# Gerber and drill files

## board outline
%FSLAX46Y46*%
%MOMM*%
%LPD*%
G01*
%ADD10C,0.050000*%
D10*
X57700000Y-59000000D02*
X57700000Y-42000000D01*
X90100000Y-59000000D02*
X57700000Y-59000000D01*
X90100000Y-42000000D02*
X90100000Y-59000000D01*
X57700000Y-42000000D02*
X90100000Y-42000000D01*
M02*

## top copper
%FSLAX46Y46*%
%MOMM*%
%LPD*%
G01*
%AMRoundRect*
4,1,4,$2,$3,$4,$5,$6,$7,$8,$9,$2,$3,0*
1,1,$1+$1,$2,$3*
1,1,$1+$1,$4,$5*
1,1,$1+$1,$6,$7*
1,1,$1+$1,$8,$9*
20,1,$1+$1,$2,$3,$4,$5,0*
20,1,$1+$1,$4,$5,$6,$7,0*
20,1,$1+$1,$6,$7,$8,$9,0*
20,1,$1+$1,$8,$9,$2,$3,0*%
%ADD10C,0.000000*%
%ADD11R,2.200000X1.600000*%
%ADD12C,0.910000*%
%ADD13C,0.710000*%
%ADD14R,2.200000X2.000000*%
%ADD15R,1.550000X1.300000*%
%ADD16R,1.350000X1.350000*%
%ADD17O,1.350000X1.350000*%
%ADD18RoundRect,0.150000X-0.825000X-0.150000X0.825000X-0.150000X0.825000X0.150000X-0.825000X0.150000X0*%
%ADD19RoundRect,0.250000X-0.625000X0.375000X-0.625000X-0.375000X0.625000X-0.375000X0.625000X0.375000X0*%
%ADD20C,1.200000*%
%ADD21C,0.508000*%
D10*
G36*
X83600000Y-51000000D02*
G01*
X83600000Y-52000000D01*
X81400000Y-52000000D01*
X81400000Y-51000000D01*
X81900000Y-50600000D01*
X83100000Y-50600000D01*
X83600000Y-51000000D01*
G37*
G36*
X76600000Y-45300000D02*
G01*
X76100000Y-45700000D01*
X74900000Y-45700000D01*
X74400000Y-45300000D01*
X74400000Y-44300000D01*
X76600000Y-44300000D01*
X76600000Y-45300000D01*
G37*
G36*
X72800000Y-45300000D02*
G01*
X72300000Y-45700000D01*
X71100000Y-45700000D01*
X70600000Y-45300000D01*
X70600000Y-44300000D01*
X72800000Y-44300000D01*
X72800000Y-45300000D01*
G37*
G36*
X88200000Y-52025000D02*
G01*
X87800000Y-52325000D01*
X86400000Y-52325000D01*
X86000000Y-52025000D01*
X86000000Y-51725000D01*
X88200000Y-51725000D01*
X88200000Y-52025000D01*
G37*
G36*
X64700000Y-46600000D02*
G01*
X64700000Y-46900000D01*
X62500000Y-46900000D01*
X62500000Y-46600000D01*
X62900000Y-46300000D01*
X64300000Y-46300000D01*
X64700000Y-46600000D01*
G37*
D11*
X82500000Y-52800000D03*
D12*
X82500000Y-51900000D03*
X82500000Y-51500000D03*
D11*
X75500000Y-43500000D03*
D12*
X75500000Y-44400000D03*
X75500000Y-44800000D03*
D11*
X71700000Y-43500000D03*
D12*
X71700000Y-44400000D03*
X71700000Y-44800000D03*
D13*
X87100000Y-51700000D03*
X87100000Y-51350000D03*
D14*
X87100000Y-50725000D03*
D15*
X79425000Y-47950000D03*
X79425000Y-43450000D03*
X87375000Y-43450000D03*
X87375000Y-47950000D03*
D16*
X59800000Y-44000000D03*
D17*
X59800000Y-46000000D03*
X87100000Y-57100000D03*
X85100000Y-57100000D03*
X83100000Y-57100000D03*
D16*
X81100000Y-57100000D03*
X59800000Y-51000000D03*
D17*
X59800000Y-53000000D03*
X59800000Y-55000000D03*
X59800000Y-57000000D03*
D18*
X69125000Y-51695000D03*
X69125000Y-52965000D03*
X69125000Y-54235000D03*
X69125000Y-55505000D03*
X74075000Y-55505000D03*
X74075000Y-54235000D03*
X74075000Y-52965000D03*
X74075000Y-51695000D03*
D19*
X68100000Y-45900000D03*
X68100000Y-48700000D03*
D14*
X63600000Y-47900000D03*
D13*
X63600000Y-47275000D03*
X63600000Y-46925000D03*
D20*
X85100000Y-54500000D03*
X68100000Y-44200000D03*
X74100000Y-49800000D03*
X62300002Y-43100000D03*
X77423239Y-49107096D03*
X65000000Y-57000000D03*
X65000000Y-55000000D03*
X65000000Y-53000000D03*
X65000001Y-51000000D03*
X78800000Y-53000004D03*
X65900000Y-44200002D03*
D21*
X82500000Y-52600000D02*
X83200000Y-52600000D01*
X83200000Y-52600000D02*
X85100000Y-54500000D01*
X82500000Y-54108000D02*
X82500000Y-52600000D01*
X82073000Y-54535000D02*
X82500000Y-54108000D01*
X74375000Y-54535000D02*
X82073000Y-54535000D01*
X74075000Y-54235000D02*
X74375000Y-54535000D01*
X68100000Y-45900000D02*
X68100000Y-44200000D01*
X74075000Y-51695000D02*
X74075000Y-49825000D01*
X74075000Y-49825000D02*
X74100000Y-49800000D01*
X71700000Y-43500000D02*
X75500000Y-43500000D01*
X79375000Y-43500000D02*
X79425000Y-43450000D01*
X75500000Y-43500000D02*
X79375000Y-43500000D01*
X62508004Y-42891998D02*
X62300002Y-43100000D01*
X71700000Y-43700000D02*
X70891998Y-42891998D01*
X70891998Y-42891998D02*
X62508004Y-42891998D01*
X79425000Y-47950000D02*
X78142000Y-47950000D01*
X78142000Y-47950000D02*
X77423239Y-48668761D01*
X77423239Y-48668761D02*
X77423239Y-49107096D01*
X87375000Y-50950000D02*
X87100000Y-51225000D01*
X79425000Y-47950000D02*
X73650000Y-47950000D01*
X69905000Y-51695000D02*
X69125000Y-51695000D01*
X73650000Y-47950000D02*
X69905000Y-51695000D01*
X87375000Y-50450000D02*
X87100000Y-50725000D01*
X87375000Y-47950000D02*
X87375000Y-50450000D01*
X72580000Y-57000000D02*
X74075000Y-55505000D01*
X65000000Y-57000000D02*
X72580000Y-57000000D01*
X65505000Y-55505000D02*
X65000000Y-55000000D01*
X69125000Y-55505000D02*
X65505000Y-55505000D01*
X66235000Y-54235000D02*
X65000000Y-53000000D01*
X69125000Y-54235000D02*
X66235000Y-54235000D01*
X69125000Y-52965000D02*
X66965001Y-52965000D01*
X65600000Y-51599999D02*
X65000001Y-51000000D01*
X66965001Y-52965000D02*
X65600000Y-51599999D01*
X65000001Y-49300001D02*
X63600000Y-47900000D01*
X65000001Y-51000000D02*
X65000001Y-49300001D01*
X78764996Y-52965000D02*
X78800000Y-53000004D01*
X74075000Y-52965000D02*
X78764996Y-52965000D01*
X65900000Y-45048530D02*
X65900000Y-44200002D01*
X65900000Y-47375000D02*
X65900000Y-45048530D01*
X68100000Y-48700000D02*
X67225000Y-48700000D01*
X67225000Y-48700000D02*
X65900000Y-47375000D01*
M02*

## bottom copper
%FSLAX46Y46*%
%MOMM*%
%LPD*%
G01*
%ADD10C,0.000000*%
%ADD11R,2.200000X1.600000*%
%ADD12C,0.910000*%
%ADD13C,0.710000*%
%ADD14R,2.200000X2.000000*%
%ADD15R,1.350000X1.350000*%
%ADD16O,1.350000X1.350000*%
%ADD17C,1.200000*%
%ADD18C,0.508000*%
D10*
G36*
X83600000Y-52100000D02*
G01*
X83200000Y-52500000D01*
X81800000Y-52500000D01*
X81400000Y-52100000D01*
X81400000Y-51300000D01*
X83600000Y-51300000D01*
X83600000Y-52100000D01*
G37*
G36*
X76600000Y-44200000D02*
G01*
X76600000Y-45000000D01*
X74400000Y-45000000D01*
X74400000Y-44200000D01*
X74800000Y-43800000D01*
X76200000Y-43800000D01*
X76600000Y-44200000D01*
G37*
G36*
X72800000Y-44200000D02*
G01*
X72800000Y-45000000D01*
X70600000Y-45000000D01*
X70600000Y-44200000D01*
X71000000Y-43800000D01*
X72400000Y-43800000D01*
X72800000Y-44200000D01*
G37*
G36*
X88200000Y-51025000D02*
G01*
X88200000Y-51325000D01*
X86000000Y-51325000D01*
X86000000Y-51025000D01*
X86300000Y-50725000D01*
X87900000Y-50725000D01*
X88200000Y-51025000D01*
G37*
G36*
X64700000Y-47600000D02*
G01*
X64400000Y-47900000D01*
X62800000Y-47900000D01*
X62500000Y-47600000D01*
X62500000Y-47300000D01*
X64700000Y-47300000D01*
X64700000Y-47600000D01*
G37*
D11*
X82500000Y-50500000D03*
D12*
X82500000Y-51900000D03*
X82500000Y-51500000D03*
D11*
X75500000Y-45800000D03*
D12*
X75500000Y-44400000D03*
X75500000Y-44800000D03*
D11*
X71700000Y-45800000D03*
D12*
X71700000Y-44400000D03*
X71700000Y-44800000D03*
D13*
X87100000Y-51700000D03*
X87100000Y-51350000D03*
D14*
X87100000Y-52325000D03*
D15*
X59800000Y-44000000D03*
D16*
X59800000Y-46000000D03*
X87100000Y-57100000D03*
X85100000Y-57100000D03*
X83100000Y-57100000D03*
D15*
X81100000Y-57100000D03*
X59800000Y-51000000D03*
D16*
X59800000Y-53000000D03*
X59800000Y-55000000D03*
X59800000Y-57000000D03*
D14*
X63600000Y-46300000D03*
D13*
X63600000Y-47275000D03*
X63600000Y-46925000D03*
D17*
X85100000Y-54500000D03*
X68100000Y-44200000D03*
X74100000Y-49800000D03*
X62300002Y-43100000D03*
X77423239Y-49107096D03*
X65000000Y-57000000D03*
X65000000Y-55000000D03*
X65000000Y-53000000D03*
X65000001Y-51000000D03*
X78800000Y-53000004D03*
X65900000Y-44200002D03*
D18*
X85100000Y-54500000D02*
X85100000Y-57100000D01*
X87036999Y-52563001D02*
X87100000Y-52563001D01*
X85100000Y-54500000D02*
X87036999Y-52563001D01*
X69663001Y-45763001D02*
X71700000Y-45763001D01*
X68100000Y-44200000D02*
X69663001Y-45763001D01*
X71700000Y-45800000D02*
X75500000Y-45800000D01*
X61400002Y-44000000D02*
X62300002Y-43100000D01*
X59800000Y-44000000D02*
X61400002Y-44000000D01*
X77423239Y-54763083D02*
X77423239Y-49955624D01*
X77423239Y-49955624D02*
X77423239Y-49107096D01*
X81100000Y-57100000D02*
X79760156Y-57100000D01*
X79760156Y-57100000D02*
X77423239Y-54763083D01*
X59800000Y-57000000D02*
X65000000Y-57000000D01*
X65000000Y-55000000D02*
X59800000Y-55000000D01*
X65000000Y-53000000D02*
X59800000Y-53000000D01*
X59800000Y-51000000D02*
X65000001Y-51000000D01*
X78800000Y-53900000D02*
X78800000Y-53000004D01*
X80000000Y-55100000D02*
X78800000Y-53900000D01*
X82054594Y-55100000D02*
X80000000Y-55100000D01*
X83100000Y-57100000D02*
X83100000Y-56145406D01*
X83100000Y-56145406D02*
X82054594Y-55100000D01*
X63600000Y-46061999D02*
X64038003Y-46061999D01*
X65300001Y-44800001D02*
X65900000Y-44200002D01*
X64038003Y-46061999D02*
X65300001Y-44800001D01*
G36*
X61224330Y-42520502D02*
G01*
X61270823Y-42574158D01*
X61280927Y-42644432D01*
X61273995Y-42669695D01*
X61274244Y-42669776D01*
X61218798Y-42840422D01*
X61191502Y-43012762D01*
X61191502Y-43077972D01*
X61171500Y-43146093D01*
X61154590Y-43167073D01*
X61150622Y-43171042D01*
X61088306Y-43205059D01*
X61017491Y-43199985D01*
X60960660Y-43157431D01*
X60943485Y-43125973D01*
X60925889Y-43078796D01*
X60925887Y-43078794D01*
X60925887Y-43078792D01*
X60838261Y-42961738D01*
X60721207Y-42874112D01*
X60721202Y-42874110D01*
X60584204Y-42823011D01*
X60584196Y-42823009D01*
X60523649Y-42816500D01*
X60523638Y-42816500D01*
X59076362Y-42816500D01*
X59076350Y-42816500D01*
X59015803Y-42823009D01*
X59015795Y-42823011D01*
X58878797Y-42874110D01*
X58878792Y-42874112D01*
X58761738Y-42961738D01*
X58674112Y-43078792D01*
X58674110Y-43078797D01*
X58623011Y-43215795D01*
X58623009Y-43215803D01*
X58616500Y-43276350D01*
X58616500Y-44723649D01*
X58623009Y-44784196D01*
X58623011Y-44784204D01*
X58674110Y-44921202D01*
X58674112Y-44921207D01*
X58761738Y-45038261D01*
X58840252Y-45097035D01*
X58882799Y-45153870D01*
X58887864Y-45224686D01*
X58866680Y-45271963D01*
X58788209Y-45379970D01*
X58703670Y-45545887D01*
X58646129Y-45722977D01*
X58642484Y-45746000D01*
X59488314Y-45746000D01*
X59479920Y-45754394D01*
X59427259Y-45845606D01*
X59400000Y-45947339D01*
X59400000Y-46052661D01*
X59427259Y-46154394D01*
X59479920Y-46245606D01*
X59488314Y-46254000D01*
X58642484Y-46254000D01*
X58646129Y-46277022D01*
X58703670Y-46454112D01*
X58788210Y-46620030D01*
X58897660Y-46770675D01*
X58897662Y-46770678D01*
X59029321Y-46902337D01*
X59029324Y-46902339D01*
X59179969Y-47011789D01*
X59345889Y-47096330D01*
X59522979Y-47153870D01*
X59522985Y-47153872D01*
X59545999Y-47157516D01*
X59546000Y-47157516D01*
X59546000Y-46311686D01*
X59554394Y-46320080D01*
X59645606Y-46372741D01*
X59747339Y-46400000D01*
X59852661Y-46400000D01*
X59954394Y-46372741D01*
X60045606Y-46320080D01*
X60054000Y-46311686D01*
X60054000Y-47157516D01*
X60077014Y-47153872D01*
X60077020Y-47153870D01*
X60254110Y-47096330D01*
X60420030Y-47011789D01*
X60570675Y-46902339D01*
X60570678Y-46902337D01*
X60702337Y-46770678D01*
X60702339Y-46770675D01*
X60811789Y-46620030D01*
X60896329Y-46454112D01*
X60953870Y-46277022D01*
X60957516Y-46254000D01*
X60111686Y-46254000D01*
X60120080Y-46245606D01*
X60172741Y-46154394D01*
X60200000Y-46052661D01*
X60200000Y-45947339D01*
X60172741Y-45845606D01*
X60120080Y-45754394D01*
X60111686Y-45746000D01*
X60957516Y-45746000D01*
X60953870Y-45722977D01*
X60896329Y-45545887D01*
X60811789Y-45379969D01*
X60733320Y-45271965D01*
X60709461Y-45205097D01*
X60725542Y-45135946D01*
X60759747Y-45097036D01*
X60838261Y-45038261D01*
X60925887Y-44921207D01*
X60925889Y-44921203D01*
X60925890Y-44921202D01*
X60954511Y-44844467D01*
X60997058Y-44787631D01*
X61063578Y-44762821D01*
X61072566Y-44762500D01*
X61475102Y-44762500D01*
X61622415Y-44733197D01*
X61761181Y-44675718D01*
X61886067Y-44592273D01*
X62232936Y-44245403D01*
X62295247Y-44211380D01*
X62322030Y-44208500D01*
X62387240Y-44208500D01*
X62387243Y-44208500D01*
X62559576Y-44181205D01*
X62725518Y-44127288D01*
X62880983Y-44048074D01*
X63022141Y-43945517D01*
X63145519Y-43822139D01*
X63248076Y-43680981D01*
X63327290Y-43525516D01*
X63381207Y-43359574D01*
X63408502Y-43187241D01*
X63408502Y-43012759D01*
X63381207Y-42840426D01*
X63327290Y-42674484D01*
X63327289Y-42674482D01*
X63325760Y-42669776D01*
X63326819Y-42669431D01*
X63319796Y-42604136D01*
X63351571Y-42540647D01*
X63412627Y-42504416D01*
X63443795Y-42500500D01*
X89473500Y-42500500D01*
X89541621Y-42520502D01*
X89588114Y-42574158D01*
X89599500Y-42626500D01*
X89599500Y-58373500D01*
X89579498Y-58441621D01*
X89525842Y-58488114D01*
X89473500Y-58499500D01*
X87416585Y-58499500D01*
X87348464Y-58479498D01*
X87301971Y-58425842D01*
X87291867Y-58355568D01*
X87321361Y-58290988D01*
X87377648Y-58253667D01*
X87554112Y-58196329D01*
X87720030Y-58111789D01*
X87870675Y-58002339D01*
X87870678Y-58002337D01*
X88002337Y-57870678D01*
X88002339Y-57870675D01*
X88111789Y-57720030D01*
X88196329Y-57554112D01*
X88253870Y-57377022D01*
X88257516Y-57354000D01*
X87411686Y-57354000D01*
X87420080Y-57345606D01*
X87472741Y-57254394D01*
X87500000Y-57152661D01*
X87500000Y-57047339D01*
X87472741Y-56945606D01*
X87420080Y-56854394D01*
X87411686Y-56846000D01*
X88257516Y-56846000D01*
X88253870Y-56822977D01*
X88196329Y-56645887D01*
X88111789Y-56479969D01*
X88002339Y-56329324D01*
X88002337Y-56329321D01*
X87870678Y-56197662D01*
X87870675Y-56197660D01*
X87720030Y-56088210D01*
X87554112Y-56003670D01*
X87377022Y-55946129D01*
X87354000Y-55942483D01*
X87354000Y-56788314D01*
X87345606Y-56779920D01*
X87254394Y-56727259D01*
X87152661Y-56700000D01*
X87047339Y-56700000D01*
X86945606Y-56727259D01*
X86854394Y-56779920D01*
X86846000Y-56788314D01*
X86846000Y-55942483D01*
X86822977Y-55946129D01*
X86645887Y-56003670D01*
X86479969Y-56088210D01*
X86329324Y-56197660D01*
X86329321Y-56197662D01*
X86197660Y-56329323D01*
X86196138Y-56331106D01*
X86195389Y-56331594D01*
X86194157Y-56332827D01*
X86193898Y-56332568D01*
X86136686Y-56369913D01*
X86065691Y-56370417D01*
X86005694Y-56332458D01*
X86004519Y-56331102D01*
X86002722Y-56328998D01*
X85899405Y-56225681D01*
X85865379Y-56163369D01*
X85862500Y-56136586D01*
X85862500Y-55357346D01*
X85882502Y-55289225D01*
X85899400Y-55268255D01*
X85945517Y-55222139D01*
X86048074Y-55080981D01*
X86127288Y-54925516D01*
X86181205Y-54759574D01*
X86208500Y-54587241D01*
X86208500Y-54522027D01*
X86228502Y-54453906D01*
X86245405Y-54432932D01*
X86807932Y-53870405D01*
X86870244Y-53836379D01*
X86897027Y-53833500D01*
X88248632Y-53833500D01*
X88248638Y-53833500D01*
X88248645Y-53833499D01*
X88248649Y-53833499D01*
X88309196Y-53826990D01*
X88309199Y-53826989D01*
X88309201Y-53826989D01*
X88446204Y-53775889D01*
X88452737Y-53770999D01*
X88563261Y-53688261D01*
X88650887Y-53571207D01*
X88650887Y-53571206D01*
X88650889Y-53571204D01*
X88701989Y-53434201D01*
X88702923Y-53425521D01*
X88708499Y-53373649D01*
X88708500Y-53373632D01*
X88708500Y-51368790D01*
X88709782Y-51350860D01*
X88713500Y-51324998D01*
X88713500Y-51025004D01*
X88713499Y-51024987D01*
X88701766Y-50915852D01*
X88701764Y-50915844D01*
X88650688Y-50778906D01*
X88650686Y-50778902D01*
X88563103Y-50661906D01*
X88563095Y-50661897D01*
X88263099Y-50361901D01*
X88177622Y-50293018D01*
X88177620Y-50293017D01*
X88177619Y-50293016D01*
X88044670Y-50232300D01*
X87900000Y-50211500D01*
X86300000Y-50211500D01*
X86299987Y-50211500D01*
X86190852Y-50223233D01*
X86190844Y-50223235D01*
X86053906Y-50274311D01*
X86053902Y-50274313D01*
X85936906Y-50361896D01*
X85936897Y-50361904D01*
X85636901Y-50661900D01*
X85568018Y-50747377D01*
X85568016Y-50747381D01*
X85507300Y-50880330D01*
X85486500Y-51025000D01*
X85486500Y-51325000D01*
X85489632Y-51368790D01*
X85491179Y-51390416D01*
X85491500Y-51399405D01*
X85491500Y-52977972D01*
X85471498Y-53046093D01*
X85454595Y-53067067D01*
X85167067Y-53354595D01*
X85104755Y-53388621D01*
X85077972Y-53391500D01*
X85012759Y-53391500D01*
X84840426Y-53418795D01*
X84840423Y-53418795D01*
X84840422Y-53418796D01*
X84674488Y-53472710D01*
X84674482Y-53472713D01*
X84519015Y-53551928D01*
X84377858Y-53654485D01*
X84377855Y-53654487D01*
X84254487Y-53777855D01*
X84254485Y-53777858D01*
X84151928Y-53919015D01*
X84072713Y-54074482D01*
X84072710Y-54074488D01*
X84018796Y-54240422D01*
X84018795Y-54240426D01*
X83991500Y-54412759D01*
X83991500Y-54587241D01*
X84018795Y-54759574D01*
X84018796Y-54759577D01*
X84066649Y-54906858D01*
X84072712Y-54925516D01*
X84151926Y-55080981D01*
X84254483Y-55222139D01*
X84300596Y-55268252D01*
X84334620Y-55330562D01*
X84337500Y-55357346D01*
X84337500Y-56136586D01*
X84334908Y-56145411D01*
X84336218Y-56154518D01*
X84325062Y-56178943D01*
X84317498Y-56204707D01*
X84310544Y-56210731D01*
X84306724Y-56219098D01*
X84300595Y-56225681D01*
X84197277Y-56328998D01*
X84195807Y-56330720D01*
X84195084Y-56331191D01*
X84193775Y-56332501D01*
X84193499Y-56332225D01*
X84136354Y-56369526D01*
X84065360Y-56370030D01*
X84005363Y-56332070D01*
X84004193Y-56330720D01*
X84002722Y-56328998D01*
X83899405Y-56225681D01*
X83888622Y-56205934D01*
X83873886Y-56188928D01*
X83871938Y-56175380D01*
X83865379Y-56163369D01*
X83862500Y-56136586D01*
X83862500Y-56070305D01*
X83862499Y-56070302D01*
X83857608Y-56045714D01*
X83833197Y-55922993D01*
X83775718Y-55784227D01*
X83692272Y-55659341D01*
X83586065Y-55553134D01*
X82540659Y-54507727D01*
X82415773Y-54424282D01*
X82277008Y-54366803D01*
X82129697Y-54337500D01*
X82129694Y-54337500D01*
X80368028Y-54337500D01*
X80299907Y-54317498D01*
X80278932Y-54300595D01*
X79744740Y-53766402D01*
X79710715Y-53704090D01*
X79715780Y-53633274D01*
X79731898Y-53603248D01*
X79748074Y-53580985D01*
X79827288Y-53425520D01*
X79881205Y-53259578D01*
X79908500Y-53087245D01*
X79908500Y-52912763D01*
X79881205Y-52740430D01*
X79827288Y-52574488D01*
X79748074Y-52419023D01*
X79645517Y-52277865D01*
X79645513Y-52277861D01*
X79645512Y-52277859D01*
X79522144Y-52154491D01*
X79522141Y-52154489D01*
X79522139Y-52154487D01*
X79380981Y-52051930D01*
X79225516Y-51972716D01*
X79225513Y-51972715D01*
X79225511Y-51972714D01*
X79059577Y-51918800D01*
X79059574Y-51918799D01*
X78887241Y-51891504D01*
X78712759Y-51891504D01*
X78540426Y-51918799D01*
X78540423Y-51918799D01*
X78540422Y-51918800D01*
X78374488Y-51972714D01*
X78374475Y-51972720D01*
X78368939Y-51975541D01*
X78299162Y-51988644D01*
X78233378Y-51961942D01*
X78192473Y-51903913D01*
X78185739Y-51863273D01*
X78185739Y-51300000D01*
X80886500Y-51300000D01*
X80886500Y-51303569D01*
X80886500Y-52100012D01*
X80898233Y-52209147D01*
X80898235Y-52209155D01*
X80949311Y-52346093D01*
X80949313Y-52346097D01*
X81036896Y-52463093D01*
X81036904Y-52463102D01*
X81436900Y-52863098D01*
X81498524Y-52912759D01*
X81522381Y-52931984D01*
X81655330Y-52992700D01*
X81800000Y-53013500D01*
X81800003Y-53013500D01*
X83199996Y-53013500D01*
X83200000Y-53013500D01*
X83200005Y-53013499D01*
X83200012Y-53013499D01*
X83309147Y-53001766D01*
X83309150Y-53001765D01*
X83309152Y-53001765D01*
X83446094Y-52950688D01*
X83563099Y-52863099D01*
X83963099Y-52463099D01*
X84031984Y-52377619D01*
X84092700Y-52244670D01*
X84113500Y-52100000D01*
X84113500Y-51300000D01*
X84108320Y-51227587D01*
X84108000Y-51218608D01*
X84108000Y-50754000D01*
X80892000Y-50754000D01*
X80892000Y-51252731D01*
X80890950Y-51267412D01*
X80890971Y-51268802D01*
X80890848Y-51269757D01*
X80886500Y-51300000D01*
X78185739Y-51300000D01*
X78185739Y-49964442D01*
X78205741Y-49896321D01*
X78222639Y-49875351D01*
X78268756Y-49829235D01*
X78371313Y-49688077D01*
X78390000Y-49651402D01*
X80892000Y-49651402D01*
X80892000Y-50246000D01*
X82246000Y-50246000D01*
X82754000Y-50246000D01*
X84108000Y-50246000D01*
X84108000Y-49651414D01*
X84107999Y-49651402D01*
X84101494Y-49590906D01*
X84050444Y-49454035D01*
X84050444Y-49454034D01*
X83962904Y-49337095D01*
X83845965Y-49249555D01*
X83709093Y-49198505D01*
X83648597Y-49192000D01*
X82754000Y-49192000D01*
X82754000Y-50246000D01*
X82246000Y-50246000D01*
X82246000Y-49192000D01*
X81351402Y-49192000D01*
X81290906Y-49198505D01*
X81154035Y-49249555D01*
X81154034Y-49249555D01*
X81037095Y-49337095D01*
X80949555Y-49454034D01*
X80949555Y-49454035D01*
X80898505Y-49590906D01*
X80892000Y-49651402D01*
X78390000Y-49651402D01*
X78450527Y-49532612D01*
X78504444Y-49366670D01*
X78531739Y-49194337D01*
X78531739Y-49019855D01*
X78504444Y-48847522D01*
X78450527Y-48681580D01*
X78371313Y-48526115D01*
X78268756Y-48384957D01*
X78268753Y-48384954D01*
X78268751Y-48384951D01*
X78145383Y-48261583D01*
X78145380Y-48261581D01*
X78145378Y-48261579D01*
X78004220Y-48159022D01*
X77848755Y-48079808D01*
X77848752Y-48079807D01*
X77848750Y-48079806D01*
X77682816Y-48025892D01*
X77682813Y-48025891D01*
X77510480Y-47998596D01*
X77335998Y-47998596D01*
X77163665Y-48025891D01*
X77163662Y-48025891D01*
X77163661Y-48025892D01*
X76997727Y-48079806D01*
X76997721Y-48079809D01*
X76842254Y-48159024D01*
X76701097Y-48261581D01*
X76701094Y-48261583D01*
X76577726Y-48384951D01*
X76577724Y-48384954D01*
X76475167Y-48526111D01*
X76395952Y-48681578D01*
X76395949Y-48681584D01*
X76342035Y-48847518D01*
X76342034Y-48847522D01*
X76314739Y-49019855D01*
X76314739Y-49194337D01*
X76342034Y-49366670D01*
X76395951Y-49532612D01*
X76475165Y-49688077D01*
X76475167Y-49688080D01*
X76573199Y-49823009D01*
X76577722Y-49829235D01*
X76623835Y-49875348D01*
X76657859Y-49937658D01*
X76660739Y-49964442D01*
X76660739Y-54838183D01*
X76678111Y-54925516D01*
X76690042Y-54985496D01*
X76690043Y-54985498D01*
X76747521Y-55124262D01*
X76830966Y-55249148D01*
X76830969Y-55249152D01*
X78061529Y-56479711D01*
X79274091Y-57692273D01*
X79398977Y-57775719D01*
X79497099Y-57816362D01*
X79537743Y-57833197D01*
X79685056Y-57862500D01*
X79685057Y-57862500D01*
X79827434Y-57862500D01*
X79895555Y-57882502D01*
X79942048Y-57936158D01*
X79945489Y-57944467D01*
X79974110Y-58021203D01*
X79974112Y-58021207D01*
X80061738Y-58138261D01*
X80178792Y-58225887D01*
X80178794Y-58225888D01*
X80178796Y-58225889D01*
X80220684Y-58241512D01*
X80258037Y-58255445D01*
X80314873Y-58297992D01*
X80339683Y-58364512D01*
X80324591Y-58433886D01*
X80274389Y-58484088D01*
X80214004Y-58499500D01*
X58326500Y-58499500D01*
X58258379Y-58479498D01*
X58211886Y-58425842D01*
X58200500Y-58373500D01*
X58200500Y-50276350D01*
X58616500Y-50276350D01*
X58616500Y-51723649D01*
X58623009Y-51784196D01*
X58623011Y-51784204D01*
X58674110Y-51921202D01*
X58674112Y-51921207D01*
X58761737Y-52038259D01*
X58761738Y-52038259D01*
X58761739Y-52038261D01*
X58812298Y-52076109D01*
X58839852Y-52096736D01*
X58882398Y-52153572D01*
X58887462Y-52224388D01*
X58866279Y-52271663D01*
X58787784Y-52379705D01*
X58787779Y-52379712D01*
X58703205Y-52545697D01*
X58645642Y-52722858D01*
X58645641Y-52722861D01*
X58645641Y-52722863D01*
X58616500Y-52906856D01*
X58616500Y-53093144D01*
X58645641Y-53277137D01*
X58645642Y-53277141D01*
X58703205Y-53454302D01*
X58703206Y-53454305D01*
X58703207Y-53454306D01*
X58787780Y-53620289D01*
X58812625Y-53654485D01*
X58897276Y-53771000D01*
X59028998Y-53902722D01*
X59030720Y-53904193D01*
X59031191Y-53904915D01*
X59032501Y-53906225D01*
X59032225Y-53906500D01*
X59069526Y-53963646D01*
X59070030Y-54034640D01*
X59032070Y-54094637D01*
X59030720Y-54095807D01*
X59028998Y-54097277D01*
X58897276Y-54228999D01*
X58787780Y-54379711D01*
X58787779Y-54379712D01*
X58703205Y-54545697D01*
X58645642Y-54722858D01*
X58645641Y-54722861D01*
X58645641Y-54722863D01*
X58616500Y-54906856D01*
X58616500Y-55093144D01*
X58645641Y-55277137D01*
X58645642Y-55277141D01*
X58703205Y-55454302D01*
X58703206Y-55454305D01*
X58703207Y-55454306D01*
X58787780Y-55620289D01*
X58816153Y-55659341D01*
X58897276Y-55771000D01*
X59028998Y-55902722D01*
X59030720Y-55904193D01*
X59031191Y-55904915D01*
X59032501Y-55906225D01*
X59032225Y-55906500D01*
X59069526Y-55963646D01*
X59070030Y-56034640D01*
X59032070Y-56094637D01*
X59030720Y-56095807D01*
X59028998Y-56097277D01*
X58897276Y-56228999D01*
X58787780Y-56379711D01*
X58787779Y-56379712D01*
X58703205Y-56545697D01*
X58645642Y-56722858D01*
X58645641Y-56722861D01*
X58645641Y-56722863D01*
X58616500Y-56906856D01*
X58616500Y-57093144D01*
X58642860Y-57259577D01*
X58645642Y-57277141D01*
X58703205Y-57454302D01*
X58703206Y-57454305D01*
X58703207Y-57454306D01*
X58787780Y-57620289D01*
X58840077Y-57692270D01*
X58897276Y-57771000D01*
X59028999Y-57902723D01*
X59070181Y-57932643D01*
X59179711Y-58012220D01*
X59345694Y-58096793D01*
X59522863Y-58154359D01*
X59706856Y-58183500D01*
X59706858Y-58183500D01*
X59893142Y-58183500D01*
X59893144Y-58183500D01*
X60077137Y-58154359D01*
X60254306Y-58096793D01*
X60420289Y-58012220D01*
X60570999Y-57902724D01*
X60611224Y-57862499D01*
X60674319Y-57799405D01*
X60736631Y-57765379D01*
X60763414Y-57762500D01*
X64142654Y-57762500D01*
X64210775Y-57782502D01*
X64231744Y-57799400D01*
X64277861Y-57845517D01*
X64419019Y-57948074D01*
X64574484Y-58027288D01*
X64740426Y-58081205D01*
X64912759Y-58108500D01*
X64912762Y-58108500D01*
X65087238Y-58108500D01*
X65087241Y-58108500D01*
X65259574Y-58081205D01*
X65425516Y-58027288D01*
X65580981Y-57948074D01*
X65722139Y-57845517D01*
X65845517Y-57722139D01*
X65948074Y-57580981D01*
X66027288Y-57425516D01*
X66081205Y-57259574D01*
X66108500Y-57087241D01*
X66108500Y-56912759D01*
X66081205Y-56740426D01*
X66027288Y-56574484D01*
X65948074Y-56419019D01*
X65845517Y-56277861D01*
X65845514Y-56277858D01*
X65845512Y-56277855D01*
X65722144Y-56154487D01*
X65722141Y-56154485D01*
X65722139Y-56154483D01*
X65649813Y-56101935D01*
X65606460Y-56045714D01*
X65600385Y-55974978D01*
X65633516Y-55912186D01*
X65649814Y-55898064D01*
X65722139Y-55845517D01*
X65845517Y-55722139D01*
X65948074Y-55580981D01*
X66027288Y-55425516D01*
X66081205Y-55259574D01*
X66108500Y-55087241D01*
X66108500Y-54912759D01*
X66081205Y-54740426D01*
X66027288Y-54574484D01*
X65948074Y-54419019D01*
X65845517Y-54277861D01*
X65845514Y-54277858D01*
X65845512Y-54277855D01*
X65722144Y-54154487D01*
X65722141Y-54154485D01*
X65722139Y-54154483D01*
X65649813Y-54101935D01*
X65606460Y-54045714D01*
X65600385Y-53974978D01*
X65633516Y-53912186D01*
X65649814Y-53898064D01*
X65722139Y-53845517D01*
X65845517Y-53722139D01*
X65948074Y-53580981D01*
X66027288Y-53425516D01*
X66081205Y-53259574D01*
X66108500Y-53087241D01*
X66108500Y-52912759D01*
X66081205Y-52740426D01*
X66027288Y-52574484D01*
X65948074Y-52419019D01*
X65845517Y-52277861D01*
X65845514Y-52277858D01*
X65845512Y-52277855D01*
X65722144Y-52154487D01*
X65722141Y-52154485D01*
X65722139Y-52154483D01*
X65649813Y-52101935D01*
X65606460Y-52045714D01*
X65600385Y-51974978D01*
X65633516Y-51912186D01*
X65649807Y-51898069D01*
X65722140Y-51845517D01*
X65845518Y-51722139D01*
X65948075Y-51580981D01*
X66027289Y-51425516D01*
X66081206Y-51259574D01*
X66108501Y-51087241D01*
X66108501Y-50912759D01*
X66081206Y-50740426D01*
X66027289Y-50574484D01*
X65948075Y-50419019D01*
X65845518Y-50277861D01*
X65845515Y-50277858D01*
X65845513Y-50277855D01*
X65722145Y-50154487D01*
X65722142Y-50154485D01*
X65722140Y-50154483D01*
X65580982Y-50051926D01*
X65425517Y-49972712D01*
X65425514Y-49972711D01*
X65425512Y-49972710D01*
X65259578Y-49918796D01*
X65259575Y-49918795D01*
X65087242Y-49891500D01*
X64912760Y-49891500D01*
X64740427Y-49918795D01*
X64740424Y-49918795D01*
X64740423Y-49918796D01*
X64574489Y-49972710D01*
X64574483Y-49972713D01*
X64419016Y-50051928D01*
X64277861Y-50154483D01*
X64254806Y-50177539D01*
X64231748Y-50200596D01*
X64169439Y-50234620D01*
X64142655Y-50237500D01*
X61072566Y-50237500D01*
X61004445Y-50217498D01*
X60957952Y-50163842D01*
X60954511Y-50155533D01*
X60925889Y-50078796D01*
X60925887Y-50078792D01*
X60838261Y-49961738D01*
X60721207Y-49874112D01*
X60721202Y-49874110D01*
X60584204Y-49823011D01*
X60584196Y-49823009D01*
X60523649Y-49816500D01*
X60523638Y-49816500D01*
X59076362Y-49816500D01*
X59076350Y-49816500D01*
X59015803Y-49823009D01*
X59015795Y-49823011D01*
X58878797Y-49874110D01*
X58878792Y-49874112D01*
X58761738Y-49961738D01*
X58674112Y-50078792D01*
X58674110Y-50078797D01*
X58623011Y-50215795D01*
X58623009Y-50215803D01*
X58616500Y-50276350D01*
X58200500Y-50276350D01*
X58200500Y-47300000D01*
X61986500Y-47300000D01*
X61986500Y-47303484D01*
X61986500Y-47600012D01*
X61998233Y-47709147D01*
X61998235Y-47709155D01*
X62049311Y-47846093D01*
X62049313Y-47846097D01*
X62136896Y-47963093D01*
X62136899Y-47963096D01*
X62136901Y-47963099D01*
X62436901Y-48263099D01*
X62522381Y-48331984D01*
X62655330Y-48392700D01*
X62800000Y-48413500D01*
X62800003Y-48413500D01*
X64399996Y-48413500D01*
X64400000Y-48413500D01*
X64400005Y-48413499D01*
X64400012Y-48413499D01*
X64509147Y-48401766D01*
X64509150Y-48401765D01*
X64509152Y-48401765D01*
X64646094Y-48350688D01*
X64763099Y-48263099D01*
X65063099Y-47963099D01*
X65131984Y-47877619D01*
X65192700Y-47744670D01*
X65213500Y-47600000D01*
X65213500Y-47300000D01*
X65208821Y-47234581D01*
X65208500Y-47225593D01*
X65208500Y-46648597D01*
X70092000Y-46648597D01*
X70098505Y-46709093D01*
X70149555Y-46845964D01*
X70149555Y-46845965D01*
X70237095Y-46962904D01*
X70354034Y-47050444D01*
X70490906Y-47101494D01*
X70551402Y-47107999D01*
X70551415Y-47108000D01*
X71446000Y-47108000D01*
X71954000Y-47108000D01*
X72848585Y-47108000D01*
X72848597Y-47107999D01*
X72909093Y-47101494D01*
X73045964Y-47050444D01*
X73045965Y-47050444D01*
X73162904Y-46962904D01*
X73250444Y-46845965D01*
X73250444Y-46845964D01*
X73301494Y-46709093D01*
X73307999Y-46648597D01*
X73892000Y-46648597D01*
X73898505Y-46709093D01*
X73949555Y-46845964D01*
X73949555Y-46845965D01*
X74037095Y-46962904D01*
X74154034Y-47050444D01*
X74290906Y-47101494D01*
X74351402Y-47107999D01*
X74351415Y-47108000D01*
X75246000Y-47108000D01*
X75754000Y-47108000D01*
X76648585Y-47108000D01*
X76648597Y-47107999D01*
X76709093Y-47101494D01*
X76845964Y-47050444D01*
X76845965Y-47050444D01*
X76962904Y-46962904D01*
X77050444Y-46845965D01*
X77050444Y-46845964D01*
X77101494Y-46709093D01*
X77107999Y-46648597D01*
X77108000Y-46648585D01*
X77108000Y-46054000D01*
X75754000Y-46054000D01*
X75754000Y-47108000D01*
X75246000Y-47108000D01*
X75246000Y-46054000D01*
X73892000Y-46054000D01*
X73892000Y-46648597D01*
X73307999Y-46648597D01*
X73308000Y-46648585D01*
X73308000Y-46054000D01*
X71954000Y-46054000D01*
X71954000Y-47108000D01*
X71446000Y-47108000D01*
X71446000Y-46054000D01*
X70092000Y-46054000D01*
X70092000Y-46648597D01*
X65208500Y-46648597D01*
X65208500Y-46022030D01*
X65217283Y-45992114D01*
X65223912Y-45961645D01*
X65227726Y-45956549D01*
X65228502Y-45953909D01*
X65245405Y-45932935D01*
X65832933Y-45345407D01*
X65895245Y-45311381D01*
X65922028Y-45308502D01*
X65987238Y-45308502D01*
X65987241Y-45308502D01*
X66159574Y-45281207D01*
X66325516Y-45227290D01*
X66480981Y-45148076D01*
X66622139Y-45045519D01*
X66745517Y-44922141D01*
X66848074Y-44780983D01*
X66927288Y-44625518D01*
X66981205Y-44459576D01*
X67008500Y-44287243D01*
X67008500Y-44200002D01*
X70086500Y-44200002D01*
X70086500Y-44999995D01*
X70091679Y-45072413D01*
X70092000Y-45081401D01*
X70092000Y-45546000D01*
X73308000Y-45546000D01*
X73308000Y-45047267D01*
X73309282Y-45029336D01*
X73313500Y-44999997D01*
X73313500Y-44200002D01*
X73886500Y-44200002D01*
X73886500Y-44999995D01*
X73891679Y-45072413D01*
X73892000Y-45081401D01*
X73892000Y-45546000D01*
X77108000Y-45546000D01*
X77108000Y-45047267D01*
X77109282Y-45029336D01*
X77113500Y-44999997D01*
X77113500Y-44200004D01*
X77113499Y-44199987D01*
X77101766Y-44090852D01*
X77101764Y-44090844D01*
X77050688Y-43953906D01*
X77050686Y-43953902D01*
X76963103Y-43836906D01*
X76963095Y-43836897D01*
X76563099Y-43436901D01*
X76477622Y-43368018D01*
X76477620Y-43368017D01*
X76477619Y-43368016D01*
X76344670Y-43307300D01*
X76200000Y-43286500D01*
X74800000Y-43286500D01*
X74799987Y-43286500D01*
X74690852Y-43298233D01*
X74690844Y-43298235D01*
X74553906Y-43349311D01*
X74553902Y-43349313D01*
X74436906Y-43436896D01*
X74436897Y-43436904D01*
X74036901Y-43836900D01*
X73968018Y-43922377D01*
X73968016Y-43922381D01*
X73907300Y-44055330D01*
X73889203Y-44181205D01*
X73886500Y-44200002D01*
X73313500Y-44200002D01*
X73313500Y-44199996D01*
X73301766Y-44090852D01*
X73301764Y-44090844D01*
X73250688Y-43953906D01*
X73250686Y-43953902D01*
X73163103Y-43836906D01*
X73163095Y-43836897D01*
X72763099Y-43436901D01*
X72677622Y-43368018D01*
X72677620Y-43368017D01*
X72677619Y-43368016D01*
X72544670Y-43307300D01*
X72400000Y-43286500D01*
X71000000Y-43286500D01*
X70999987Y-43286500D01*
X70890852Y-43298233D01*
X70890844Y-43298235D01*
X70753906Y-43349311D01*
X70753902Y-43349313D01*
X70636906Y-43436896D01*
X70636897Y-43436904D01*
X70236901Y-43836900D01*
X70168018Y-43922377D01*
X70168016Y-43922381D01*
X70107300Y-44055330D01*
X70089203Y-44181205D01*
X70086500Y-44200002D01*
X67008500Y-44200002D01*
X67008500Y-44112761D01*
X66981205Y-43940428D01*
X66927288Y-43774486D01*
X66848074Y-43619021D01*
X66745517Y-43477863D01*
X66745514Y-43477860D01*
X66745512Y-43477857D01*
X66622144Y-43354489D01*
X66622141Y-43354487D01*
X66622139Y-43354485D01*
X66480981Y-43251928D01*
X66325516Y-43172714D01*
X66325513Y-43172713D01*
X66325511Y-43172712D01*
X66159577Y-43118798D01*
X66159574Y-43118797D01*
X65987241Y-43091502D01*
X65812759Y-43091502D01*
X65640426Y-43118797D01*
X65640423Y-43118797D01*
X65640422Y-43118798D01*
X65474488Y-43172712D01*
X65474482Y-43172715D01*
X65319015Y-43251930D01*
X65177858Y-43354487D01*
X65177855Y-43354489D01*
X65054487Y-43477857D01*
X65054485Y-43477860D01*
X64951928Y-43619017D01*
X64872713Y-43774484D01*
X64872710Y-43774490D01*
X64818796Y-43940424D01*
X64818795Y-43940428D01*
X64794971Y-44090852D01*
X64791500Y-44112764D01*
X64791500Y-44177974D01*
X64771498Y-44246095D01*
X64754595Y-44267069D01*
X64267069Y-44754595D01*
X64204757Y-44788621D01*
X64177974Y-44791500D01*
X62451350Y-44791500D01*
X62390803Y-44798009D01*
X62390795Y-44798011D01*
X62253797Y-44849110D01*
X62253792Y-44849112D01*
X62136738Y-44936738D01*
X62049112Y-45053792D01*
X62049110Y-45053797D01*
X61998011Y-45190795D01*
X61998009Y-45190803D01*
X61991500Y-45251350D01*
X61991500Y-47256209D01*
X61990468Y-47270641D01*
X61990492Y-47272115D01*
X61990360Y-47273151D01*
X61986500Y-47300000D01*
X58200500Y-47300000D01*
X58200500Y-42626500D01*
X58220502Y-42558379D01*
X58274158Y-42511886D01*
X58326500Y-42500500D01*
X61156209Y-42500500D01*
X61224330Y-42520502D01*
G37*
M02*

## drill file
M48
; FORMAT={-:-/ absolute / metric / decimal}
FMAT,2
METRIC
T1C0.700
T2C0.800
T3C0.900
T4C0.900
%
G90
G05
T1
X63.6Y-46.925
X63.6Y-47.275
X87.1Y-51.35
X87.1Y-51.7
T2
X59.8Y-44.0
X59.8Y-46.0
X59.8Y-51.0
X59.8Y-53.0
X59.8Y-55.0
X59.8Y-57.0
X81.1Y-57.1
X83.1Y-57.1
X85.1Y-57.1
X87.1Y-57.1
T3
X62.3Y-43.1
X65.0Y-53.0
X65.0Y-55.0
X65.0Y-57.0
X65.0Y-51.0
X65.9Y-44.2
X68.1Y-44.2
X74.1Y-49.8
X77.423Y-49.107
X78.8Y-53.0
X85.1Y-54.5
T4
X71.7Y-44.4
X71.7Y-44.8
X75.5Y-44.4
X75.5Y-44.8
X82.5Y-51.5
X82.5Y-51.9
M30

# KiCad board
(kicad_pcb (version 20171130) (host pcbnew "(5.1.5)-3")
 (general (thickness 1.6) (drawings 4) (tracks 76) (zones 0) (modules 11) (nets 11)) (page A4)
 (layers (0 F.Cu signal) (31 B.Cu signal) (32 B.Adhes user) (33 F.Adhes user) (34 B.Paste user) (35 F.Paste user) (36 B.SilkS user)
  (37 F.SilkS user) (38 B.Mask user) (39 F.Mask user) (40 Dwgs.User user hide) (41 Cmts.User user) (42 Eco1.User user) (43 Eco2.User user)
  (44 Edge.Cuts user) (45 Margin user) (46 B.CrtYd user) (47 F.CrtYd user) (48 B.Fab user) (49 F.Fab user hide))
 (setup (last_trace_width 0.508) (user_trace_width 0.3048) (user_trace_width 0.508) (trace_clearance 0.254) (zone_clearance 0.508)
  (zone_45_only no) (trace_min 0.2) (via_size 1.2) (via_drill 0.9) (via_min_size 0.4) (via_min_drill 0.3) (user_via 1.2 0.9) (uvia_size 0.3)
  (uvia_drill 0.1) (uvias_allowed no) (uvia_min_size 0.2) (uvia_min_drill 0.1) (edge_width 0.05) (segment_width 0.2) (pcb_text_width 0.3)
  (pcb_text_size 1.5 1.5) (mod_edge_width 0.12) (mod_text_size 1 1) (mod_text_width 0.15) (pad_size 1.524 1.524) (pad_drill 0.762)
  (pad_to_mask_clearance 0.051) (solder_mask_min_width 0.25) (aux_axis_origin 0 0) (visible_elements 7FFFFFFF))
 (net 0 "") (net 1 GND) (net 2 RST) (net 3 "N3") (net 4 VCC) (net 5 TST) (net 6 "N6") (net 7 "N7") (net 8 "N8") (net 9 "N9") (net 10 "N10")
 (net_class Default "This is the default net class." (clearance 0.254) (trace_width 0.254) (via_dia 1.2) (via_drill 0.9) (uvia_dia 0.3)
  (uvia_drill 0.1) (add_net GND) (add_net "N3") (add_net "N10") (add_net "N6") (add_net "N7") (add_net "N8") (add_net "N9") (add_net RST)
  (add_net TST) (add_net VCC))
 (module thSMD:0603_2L (layer F.Cu) (at 82.5 51.7) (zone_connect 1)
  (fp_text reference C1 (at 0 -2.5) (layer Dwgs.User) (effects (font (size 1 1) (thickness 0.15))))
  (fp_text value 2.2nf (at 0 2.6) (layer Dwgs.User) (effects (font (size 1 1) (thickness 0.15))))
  (fp_poly (pts (xy 1.1 -0.4) (xy 1.1 0.4) (xy 0.7 0.8) (xy -0.7 0.8) (xy -1.1 0.4) (xy -1.1 -0.4)) (layer B.Cu) (width 0))
  (fp_poly (pts (xy 1.1 -0.7) (xy 1.1 0.3) (xy -1.1 0.3) (xy -1.1 -0.7) (xy -0.6 -1.1) (xy 0.6 -1.1)) (layer F.Cu) (width 0))
  (pad 2 smd rect (at 0 -1.2) (size 2.2 1.6) (layers B.Cu B.Mask) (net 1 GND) (clearance 0.2) (zone_connect 1))
  (pad 1 smd rect (at 0 1.1) (size 2.2 1.6) (layers F.Cu F.Mask) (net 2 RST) (clearance 0.2) (zone_connect 1))
  (pad 1 thru_hole circle (at 0 0.2) (size 0.91 0.91) (drill 0.9) (layers *.Cu) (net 2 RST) (clearance 0.01) (zone_connect 2))
  (pad 1 thru_hole circle (at 0 -0.2) (size 0.91 0.91) (drill 0.9) (layers *.Cu) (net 2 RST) (clearance 0.01) (zone_connect 2)))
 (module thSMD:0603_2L (layer F.Cu) (at 75.5 44.6 180) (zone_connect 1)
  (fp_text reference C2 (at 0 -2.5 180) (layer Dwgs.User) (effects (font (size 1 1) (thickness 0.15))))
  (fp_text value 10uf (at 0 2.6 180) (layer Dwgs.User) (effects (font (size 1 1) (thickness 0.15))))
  (fp_poly (pts (xy 1.1 -0.4) (xy 1.1 0.4) (xy 0.7 0.8) (xy -0.7 0.8) (xy -1.1 0.4) (xy -1.1 -0.4)) (layer B.Cu) (width 0))
  (fp_poly (pts (xy 1.1 -0.7) (xy 1.1 0.3) (xy -1.1 0.3) (xy -1.1 -0.7) (xy -0.6 -1.1) (xy 0.6 -1.1)) (layer F.Cu) (width 0))
  (pad 2 smd rect (at 0 -1.2 180) (size 2.2 1.6) (layers B.Cu B.Mask) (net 1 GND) (clearance 0.2) (zone_connect 1))
  (pad 1 smd rect (at 0 1.1 180) (size 2.2 1.6) (layers F.Cu F.Mask) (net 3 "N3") (clearance 0.2) (zone_connect 1))
  (pad 1 thru_hole circle (at 0 0.2 180) (size 0.91 0.91) (drill 0.9) (layers *.Cu) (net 3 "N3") (clearance 0.01) (zone_connect 2))
  (pad 1 thru_hole circle (at 0 -0.2 180) (size 0.91 0.91) (drill 0.9) (layers *.Cu) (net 3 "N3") (clearance 0.01) (zone_connect 2)))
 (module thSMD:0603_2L (layer F.Cu) (at 71.7 44.6 180) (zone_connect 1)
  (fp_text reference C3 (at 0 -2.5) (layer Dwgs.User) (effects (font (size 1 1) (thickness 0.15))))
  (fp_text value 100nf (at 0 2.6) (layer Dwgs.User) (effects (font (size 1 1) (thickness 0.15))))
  (fp_poly (pts (xy 1.1 -0.4) (xy 1.1 0.4) (xy 0.7 0.8) (xy -0.7 0.8) (xy -1.1 0.4) (xy -1.1 -0.4)) (layer B.Cu) (width 0))
  (fp_poly (pts (xy 1.1 -0.7) (xy 1.1 0.3) (xy -1.1 0.3) (xy -1.1 -0.7) (xy -0.6 -1.1) (xy 0.6 -1.1)) (layer F.Cu) (width 0))
  (pad 2 smd rect (at 0 -1.2 180) (size 2.2 1.6) (layers B.Cu B.Mask) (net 1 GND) (clearance 0.2) (zone_connect 1))
  (pad 1 smd rect (at 0 1.1 180) (size 2.2 1.6) (layers F.Cu F.Mask) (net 3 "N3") (clearance 0.2) (zone_connect 1))
  (pad 1 thru_hole circle (at 0 0.2 180) (size 0.91 0.91) (drill 0.9) (layers *.Cu) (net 3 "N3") (clearance 0.01) (zone_connect 2))
  (pad 1 thru_hole circle (at 0 -0.2 180) (size 0.91 0.91) (drill 0.9) (layers *.Cu) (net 3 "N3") (clearance 0.01) (zone_connect 2)))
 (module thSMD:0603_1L (layer F.Cu) (at 87.1 51.525 180) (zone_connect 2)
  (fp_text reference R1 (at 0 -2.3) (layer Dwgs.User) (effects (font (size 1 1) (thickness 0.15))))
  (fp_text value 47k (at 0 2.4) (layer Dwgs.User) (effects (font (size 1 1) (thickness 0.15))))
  (fp_poly (pts (xy 1.1 -0.5) (xy 1.1 -0.2) (xy -1.1 -0.2) (xy -1.1 -0.5) (xy -0.7 -0.8) (xy 0.7 -0.8)) (layer F.Cu) (width 0))
  (fp_poly (pts (xy 1.1 0.5) (xy 0.8 0.8) (xy -0.8 0.8) (xy -1.1 0.5) (xy -1.1 0.2) (xy 1.1 0.2)) (layer B.Cu) (width 0))
  (pad 1 thru_hole circle (at 0 -0.175 180) (size 0.71 0.71) (drill 0.7) (layers *.Cu) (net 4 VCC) (clearance 0.01) (zone_connect 2))
  (pad 1 thru_hole circle (at 0 0.175 180) (size 0.71 0.71) (drill 0.7) (layers *.Cu) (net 4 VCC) (clearance 0.01) (zone_connect 2))
  (pad 2 smd rect (at 0 -0.8 180) (size 2.2 2) (layers B.Cu B.Mask) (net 2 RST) (zone_connect 0))
  (pad 1 smd rect (at 0 0.8 180) (size 2.2 2) (layers F.Cu F.Mask) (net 4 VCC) (zone_connect 0)))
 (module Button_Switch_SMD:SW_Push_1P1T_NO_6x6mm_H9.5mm (layer F.Cu) (at 83.4 45.7)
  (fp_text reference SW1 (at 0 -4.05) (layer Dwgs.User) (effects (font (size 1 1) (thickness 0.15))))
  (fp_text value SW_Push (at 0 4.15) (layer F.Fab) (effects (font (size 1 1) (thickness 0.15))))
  (pad 2 smd rect (at -3.975 2.25) (size 1.55 1.3) (layers F.Cu F.Paste F.Mask) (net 4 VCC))
  (pad 1 smd rect (at -3.975 -2.25) (size 1.55 1.3) (layers F.Cu F.Paste F.Mask) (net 3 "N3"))
  (pad 1 smd rect (at 3.975 -2.25) (size 1.55 1.3) (layers F.Cu F.Paste F.Mask) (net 3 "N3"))
  (pad 2 smd rect (at 3.975 2.25) (size 1.55 1.3) (layers F.Cu F.Paste F.Mask) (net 4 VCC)))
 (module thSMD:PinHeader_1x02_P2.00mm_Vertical (layer F.Cu) (at 59.8 44)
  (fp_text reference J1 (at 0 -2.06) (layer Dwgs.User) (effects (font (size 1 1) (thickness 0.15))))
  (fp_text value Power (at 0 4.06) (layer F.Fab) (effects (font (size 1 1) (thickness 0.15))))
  (pad 1 thru_hole rect (at 0 0) (size 1.35 1.35) (drill 0.8) (layers *.Mask B.Cu) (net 3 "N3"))
  (pad 2 thru_hole oval (at 0 2) (size 1.35 1.35) (drill 0.8) (layers *.Mask B.Cu) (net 1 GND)))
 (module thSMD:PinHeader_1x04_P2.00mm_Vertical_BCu (layer F.Cu) (at 81.1 57.1 90)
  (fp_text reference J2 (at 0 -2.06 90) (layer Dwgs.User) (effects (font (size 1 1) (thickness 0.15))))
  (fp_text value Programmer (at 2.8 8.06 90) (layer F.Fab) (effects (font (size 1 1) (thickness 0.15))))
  (pad 4 thru_hole oval (at 0 6 90) (size 1.35 1.35) (drill 0.8) (layers *.Mask B.Cu) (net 1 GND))
  (pad 3 thru_hole oval (at 0 4 90) (size 1.35 1.35) (drill 0.8) (layers *.Mask B.Cu) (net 2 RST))
  (pad 2 thru_hole oval (at 0 2 90) (size 1.35 1.35) (drill 0.8) (layers *.Mask B.Cu) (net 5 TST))
  (pad 1 thru_hole rect (at 0 0 90) (size 1.35 1.35) (drill 0.8) (layers *.Mask B.Cu) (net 4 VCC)))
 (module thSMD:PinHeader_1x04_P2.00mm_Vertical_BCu (layer F.Cu) (at 59.8 51)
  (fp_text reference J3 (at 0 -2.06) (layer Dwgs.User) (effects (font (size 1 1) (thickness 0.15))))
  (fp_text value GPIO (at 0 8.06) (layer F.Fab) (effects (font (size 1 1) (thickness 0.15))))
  (pad 1 thru_hole rect (at 0 0) (size 1.35 1.35) (drill 0.8) (layers *.Mask B.Cu) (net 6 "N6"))
  (pad 2 thru_hole oval (at 0 2) (size 1.35 1.35) (drill 0.8) (layers *.Mask B.Cu) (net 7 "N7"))
  (pad 3 thru_hole oval (at 0 4) (size 1.35 1.35) (drill 0.8) (layers *.Mask B.Cu) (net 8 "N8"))
  (pad 4 thru_hole oval (at 0 6) (size 1.35 1.35) (drill 0.8) (layers *.Mask B.Cu) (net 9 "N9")))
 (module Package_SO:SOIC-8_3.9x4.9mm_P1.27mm (layer F.Cu) (at 71.6 53.6)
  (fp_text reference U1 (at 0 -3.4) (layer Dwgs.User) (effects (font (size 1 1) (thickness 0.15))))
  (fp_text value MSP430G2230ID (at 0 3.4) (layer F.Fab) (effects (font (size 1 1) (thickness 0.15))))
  (pad 1 smd roundrect (at -2.475 -1.905) (size 1.95 0.6) (layers F.Cu F.Paste F.Mask) (roundrect_rratio 0.25) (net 4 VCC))
  (pad 2 smd roundrect (at -2.475 -0.635) (size 1.95 0.6) (layers F.Cu F.Paste F.Mask) (roundrect_rratio 0.25) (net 6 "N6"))
  (pad 3 smd roundrect (at -2.475 0.635) (size 1.95 0.6) (layers F.Cu F.Paste F.Mask) (roundrect_rratio 0.25) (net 7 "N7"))
  (pad 4 smd roundrect (at -2.475 1.905) (size 1.95 0.6) (layers F.Cu F.Paste F.Mask) (roundrect_rratio 0.25) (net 8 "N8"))
  (pad 5 smd roundrect (at 2.475 1.905) (size 1.95 0.6) (layers F.Cu F.Paste F.Mask) (roundrect_rratio 0.25) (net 9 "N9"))
  (pad 6 smd roundrect (at 2.475 0.635) (size 1.95 0.6) (layers F.Cu F.Paste F.Mask) (roundrect_rratio 0.25) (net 2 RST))
  (pad 7 smd roundrect (at 2.475 -0.635) (size 1.95 0.6) (layers F.Cu F.Paste F.Mask) (roundrect_rratio 0.25) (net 5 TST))
  (pad 8 smd roundrect (at 2.475 -1.905) (size 1.95 0.6) (layers F.Cu F.Paste F.Mask) (roundrect_rratio 0.25) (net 1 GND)))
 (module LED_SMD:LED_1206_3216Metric (layer F.Cu) (at 68.1 47.3 270)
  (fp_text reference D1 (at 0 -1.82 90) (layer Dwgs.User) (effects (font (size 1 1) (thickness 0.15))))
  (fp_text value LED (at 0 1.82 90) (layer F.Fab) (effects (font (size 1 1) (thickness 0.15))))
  (pad 1 smd roundrect (at -1.4 0 270) (size 1.25 1.75) (layers F.Cu F.Paste F.Mask) (roundrect_rratio 0.2) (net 1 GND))
  (pad 2 smd roundrect (at 1.4 0 270) (size 1.25 1.75) (layers F.Cu F.Paste F.Mask) (roundrect_rratio 0.2) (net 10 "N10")))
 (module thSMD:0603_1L (layer F.Cu) (at 63.6 47.1) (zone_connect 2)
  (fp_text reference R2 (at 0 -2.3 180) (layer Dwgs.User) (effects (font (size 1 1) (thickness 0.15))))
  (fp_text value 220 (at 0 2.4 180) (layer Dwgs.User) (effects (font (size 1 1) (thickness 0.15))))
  (fp_poly (pts (xy 1.1 0.5) (xy 0.8 0.8) (xy -0.8 0.8) (xy -1.1 0.5) (xy -1.1 0.2) (xy 1.1 0.2)) (layer B.Cu) (width 0))
  (fp_poly (pts (xy 1.1 -0.5) (xy 1.1 -0.2) (xy -1.1 -0.2) (xy -1.1 -0.5) (xy -0.7 -0.8) (xy 0.7 -0.8)) (layer F.Cu) (width 0))
  (pad 1 smd rect (at 0 0.8) (size 2.2 2) (layers F.Cu F.Mask) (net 6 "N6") (zone_connect 0))
  (pad 2 smd rect (at 0 -0.8) (size 2.2 2) (layers B.Cu B.Mask) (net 10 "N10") (zone_connect 0))
  (pad 1 thru_hole circle (at 0 0.175) (size 0.71 0.71) (drill 0.7) (layers *.Cu) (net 6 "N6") (clearance 0.01) (zone_connect 2))
  (pad 1 thru_hole circle (at 0 -0.175) (size 0.71 0.71) (drill 0.7) (layers *.Cu) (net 6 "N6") (clearance 0.01) (zone_connect 2)))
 (gr_line (start 57.7 59) (end 57.7 42) (layer Edge.Cuts) (width 0.05))
 (gr_line (start 90.1 59) (end 57.7 59) (layer Edge.Cuts) (width 0.05))
 (gr_line (start 90.1 42) (end 90.1 59) (layer Edge.Cuts) (width 0.05))
 (gr_line (start 57.7 42) (end 90.1 42) (layer Edge.Cuts) (width 0.05))
 (via (at 85.1 54.5) (size 1.2) (drill 0.9) (layers F.Cu B.Cu) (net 2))
 (segment (start 82.5 52.6) (end 83.2 52.6) (width 0.508) (layer F.Cu) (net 2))
 (segment (start 83.2 52.6) (end 85.1 54.5) (width 0.508) (layer F.Cu) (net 2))
 (segment (start 85.1 54.5) (end 85.1 57.1) (width 0.508) (layer B.Cu) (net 2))
 (segment (start 82.5 54.108) (end 82.5 52.6) (width 0.508) (layer F.Cu) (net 2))
 (segment (start 82.073 54.535) (end 82.5 54.108) (width 0.508) (layer F.Cu) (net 2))
 (segment (start 74.375 54.535) (end 82.073 54.535) (width 0.508) (layer F.Cu) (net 2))
 (segment (start 74.075 54.235) (end 74.375 54.535) (width 0.508) (layer F.Cu) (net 2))
 (segment (start 87.036999 52.563001) (end 87.1 52.563001) (width 0.508) (layer B.Cu) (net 2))
 (segment (start 85.1 54.5) (end 87.036999 52.563001) (width 0.508) (layer B.Cu) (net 2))
 (via (at 68.1 44.2) (size 1.2) (drill 0.9) (layers F.Cu B.Cu) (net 1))
 (segment (start 68.1 45.9) (end 68.1 44.2) (width 0.508) (layer F.Cu) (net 1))
 (segment (start 69.663001 45.763001) (end 71.7 45.763001) (width 0.508) (layer B.Cu) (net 1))
 (segment (start 68.1 44.2) (end 69.663001 45.763001) (width 0.508) (layer B.Cu) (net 1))
 (via (at 74.1 49.8) (size 1.2) (drill 0.9) (layers F.Cu B.Cu) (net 1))
 (segment (start 74.075 51.695) (end 74.075 49.825) (width 0.508) (layer F.Cu) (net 1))
 (segment (start 74.075 49.825) (end 74.1 49.8) (width 0.508) (layer F.Cu) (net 1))
 (segment (start 71.7 45.8) (end 75.5 45.8) (width 0.508) (layer B.Cu) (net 1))
 (via (at 62.300002 43.1) (size 1.2) (drill 0.9) (layers F.Cu B.Cu) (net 3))
 (segment (start 61.400002 44) (end 62.300002 43.1) (width 0.508) (layer B.Cu) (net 3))
 (segment (start 59.8 44) (end 61.400002 44) (width 0.508) (layer B.Cu) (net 3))
 (segment (start 71.7 43.5) (end 75.5 43.5) (width 0.508) (layer F.Cu) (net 3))
 (segment (start 79.375 43.5) (end 79.425 43.45) (width 0.508) (layer F.Cu) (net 3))
 (segment (start 75.5 43.5) (end 79.375 43.5) (width 0.508) (layer F.Cu) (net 3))
 (segment (start 62.508004 42.891998) (end 62.300002 43.1) (width 0.508) (layer F.Cu) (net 3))
 (segment (start 71.7 43.7) (end 70.891998 42.891998) (width 0.508) (layer F.Cu) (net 3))
 (segment (start 70.891998 42.891998) (end 62.508004 42.891998) (width 0.508) (layer F.Cu) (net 3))
 (segment (start 79.425 47.95) (end 78.142 47.95) (width 0.508) (layer F.Cu) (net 4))
 (segment (start 78.142 47.95) (end 77.423239 48.668761) (width 0.508) (layer F.Cu) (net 4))
 (via (at 77.423239 49.107096) (size 1.2) (drill 0.9) (layers F.Cu B.Cu) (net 4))
 (segment (start 77.423239 48.668761) (end 77.423239 49.107096) (width 0.508) (layer F.Cu) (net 4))
 (segment (start 87.375 50.95) (end 87.1 51.225) (width 0.508) (layer F.Cu) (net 4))
 (segment (start 77.423239 54.763083) (end 77.423239 49.955624) (width 0.508) (layer B.Cu) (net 4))
 (segment (start 77.423239 49.955624) (end 77.423239 49.107096) (width 0.508) (layer B.Cu) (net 4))
 (segment (start 81.1 57.1) (end 79.760156 57.1) (width 0.508) (layer B.Cu) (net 4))
 (segment (start 79.760156 57.1) (end 77.423239 54.763083) (width 0.508) (layer B.Cu) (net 4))
 (segment (start 79.425 47.95) (end 73.65 47.95) (width 0.508) (layer F.Cu) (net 4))
 (segment (start 69.905 51.695) (end 69.125 51.695) (width 0.508) (layer F.Cu) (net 4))
 (segment (start 73.65 47.95) (end 69.905 51.695) (width 0.508) (layer F.Cu) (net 4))
 (segment (start 87.375 50.45) (end 87.1 50.725) (width 0.508) (layer F.Cu) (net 4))
 (segment (start 87.375 47.95) (end 87.375 50.45) (width 0.508) (layer F.Cu) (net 4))
 (via (at 65 57) (size 1.2) (drill 0.9) (layers F.Cu B.Cu) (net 9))
 (segment (start 72.58 57) (end 74.075 55.505) (width 0.508) (layer F.Cu) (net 9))
 (segment (start 65 57) (end 72.58 57) (width 0.508) (layer F.Cu) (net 9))
 (segment (start 59.8 57) (end 65 57) (width 0.508) (layer B.Cu) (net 9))
 (via (at 65 55) (size 1.2) (drill 0.9) (layers F.Cu B.Cu) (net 8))
 (segment (start 65.505 55.505) (end 65 55) (width 0.508) (layer F.Cu) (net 8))
 (segment (start 69.125 55.505) (end 65.505 55.505) (width 0.508) (layer F.Cu) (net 8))
 (segment (start 65 55) (end 59.8 55) (width 0.508) (layer B.Cu) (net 8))
 (via (at 65 53) (size 1.2) (drill 0.9) (layers F.Cu B.Cu) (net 7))
 (segment (start 66.235 54.235) (end 65 53) (width 0.508) (layer F.Cu) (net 7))
 (segment (start 69.125 54.235) (end 66.235 54.235) (width 0.508) (layer F.Cu) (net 7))
 (segment (start 65 53) (end 59.8 53) (width 0.508) (layer B.Cu) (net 7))
 (via (at 65.000001 51) (size 1.2) (drill 0.9) (layers F.Cu B.Cu) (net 6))
 (segment (start 59.8 51) (end 65.000001 51) (width 0.508) (layer B.Cu) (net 6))
 (segment (start 69.125 52.965) (end 66.965001 52.965) (width 0.508) (layer F.Cu) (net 6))
 (segment (start 65.6 51.599999) (end 65.000001 51) (width 0.508) (layer F.Cu) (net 6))
 (segment (start 66.965001 52.965) (end 65.6 51.599999) (width 0.508) (layer F.Cu) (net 6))
 (segment (start 65.000001 49.300001) (end 63.6 47.9) (width 0.508) (layer F.Cu) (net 6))
 (segment (start 65.000001 51) (end 65.000001 49.300001) (width 0.508) (layer F.Cu) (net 6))
 (via (at 78.8 53.000004) (size 1.2) (drill 0.9) (layers F.Cu B.Cu) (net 5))
 (segment (start 78.764996 52.965) (end 78.8 53.000004) (width 0.508) (layer F.Cu) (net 5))
 (segment (start 74.075 52.965) (end 78.764996 52.965) (width 0.508) (layer F.Cu) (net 5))
 (segment (start 78.8 53.9) (end 78.8 53.000004) (width 0.508) (layer B.Cu) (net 5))
 (segment (start 80 55.1) (end 78.8 53.9) (width 0.508) (layer B.Cu) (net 5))
 (segment (start 82.054594 55.1) (end 80 55.1) (width 0.508) (layer B.Cu) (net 5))
 (segment (start 83.1 57.1) (end 83.1 56.145406) (width 0.508) (layer B.Cu) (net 5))
 (segment (start 83.1 56.145406) (end 82.054594 55.1) (width 0.508) (layer B.Cu) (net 5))
 (segment (start 65.9 45.04853) (end 65.9 44.200002) (width 0.508) (layer F.Cu) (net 10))
 (via (at 65.9 44.200002) (size 1.2) (drill 0.9) (layers F.Cu B.Cu) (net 10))
 (segment (start 63.6 46.061999) (end 64.038003 46.061999) (width 0.508) (layer B.Cu) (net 10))
 (segment (start 65.9 47.375) (end 65.9 45.04853) (width 0.508) (layer F.Cu) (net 10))
 (segment (start 65.300001 44.800001) (end 65.9 44.200002) (width 0.508) (layer B.Cu) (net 10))
 (segment (start 68.1 48.7) (end 67.225 48.7) (width 0.508) (layer F.Cu) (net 10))
 (segment (start 64.038003 46.061999) (end 65.300001 44.800001) (width 0.508) (layer B.Cu) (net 10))
 (segment (start 67.225 48.7) (end 65.9 47.375) (width 0.508) (layer F.Cu) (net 10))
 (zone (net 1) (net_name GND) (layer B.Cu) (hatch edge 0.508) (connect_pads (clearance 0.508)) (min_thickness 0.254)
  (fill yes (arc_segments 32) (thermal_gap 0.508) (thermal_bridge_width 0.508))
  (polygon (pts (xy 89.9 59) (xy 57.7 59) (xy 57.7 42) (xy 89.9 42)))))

